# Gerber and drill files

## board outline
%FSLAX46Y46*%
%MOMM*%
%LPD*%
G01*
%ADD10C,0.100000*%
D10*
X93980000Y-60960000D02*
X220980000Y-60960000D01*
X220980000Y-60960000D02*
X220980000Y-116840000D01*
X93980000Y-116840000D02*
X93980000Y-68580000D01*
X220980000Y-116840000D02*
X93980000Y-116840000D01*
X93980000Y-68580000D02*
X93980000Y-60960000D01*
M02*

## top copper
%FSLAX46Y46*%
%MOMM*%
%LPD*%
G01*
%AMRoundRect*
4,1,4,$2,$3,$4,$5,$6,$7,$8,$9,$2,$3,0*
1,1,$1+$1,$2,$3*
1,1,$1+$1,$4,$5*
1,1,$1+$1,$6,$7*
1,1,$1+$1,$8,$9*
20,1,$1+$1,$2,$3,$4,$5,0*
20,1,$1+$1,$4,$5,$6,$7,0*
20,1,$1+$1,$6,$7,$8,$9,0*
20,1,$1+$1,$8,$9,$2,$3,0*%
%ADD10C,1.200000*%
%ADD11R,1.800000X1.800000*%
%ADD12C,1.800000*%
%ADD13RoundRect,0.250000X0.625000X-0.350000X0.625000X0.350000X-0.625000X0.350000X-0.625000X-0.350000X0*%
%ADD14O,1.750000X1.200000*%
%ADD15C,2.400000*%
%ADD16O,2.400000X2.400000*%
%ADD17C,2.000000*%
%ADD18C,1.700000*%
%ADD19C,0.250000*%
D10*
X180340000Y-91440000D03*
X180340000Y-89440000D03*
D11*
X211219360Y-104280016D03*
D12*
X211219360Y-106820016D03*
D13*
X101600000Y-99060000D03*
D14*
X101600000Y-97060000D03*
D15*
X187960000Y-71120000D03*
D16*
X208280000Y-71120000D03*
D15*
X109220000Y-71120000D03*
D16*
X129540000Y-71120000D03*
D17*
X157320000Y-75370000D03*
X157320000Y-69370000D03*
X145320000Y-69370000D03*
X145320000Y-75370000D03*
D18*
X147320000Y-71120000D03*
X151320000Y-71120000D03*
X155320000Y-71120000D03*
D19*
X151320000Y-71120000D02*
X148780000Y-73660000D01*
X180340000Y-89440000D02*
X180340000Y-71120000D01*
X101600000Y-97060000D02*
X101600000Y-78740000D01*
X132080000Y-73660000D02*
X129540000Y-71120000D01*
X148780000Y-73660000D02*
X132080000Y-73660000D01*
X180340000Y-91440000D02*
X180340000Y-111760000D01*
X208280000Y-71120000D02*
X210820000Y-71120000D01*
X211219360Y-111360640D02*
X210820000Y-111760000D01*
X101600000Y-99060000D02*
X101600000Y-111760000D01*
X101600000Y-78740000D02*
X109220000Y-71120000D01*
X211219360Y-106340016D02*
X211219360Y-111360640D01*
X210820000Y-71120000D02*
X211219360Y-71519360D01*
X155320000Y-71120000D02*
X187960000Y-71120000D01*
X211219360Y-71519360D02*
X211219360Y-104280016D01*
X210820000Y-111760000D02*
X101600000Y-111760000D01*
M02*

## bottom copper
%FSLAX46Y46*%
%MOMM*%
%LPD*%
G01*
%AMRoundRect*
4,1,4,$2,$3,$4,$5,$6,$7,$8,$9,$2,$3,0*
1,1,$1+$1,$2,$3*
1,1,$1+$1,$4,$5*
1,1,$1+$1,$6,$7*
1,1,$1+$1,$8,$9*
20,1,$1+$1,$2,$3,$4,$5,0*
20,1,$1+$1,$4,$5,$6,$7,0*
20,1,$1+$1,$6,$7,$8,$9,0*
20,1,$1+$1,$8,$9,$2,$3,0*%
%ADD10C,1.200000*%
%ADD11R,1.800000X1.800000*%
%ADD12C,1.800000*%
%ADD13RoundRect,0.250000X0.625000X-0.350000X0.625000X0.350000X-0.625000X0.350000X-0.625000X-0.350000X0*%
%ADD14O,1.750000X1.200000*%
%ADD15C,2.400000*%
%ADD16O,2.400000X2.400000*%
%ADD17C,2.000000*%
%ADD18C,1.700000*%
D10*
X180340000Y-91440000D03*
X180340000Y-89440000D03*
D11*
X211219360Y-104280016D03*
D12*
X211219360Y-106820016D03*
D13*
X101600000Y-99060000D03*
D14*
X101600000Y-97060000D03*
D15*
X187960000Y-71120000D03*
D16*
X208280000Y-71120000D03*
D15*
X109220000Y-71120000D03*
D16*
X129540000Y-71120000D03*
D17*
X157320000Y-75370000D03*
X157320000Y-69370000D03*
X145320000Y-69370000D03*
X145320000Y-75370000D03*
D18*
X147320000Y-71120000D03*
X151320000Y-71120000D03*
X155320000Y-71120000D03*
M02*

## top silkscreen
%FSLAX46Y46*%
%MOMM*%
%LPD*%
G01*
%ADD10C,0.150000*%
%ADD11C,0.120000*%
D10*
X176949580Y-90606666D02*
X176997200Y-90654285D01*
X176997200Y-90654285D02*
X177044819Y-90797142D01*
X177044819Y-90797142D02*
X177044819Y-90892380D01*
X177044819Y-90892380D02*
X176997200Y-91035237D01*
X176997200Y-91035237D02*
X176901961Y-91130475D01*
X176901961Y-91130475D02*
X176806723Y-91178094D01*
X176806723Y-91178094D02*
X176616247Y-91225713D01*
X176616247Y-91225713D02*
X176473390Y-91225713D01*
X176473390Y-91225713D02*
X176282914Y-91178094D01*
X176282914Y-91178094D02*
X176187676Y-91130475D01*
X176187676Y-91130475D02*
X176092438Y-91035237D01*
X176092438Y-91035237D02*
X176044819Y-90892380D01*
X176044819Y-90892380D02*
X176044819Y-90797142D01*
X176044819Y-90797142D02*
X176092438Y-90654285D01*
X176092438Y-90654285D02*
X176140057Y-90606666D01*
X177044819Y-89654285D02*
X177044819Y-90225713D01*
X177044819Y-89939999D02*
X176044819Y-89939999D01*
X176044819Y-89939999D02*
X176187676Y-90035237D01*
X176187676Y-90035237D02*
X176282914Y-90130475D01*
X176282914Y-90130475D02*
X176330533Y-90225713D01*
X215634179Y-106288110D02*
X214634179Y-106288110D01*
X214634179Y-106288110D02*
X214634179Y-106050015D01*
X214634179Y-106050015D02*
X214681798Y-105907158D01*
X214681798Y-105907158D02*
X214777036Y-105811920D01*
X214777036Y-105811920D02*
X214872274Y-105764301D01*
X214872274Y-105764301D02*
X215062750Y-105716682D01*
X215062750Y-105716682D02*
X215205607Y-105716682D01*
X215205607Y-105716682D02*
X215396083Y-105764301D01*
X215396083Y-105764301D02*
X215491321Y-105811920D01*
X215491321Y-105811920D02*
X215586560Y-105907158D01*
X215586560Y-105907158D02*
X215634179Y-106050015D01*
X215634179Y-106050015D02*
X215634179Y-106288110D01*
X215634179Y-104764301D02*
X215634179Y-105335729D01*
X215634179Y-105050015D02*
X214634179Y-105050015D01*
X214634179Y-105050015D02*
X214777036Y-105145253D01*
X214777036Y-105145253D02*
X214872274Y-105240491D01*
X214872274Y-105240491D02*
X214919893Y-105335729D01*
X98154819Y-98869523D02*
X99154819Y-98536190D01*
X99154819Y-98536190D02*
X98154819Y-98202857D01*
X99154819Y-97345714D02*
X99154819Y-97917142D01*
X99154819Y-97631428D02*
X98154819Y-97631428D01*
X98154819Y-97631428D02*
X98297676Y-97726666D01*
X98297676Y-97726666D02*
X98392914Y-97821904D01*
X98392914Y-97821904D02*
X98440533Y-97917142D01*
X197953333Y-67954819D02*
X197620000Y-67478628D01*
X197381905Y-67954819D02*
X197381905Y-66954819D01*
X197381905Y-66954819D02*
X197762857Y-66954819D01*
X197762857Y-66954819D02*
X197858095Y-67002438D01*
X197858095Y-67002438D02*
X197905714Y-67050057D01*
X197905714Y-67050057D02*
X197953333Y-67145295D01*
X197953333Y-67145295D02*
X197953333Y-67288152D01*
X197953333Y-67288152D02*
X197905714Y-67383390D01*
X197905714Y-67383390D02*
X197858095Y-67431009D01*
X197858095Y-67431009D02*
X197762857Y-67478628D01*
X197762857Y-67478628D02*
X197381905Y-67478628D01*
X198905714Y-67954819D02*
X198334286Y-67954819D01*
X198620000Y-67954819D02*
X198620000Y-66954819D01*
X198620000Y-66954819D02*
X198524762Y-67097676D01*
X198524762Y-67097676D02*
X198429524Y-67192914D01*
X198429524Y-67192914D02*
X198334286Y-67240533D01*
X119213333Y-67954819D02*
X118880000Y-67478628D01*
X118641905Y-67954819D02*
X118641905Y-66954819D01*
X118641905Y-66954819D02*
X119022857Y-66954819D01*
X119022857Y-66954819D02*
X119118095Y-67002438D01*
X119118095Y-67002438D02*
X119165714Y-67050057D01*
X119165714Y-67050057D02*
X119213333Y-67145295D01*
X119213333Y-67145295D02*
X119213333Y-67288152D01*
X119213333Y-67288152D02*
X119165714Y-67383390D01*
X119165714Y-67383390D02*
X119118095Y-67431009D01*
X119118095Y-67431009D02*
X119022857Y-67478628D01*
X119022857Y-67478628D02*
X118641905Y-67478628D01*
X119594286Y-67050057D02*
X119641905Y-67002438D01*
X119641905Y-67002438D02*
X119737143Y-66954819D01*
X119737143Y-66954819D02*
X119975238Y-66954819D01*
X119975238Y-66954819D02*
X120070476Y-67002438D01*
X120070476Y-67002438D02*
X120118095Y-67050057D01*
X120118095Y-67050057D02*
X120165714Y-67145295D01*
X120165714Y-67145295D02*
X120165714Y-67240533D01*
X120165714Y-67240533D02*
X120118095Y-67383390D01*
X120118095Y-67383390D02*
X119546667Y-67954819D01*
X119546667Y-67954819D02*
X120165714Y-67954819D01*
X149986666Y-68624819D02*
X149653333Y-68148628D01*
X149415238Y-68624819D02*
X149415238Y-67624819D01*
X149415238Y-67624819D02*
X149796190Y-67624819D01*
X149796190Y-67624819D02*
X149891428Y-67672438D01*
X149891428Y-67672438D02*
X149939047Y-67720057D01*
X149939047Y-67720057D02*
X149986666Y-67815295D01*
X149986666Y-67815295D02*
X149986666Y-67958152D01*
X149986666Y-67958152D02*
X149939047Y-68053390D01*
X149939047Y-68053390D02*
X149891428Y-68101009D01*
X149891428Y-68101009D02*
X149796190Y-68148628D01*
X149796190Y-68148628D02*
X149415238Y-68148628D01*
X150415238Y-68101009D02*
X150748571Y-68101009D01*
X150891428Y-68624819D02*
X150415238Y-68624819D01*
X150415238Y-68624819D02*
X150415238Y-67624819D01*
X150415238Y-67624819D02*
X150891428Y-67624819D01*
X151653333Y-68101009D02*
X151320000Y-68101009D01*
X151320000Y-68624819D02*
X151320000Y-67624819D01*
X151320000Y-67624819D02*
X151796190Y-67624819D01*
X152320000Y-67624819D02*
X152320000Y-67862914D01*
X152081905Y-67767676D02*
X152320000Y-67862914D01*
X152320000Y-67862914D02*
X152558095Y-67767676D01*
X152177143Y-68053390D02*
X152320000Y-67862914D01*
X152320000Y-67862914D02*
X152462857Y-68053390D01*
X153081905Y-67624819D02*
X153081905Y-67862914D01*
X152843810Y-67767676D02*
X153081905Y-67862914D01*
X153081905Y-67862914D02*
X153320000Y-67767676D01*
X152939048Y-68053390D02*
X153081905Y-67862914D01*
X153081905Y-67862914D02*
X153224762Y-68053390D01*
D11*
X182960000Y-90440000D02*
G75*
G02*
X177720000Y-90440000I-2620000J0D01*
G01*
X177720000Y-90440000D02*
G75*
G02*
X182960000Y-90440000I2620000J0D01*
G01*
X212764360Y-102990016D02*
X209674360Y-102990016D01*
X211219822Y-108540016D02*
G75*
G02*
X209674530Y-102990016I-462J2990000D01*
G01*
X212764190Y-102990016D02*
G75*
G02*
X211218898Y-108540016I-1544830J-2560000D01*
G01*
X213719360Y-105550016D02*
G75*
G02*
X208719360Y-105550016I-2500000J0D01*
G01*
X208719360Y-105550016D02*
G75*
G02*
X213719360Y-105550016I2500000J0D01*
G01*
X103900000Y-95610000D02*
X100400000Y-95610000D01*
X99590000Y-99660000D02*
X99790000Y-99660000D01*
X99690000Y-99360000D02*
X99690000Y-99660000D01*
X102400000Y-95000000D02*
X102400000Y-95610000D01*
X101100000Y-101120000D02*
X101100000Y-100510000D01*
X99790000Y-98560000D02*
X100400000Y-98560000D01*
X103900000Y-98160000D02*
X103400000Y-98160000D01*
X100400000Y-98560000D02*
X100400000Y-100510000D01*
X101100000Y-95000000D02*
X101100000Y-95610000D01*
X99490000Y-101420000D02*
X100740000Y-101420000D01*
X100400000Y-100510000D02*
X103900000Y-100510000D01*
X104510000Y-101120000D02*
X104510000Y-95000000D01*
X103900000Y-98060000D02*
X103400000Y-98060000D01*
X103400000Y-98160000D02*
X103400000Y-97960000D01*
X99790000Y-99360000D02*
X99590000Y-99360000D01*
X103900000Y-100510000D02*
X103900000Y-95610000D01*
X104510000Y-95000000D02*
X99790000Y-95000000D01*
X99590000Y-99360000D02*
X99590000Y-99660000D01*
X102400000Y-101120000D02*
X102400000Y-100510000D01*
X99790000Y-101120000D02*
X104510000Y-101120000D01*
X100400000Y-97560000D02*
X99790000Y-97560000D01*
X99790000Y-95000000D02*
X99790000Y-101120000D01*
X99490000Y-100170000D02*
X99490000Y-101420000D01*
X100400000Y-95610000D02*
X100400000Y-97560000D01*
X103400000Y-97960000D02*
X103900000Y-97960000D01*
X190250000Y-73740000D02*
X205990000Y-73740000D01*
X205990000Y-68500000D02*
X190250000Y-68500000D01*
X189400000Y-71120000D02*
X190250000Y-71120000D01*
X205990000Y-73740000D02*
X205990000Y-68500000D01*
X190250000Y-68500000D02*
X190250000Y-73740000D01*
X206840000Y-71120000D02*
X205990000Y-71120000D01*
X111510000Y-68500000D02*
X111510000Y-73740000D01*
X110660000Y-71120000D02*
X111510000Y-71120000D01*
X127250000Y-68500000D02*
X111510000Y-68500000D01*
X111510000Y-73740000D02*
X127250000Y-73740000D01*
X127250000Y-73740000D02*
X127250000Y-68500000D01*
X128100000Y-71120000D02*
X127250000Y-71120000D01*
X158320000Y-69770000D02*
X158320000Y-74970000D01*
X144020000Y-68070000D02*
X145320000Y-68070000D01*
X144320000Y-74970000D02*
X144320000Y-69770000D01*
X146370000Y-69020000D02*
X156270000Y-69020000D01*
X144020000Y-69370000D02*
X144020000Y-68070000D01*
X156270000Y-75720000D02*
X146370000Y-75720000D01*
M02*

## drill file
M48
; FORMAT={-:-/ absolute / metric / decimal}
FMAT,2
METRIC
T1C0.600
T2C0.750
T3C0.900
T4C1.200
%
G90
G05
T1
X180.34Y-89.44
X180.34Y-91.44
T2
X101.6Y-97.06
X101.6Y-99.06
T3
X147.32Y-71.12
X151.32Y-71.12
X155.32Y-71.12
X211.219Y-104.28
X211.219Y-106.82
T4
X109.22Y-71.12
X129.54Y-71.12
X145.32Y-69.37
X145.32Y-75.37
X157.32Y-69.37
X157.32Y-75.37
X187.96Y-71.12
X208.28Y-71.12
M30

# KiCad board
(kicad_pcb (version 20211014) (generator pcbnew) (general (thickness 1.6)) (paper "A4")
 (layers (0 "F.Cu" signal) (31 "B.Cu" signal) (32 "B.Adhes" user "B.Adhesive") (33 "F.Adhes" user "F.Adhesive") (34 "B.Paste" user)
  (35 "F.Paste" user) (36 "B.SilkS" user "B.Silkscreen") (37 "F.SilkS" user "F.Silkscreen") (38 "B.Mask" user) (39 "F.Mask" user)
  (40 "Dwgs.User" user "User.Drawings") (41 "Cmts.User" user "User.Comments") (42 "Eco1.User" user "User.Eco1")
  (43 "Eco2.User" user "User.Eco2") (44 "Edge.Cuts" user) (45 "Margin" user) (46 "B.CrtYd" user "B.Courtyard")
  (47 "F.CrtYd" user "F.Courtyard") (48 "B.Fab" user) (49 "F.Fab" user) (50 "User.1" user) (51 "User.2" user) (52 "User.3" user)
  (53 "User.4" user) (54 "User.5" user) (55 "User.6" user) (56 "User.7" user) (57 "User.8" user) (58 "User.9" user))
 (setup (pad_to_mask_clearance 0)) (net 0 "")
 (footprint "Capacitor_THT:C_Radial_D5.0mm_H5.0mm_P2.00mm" (layer "F.Cu") (at 180.34 91.44 90)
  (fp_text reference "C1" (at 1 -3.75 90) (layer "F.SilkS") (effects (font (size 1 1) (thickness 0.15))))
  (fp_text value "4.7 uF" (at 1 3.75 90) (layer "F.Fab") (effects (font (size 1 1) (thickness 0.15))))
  (fp_circle (center 1 0) (end 3.62 0) (layer "F.SilkS") (width 0.12) (fill none))
  (pad "1" thru_hole circle (at 0 0 90) (size 1.2 1.2) (drill 0.6) (layers *.Cu *.Mask))
  (pad "2" thru_hole circle (at 2 0 90) (size 1.2 1.2) (drill 0.6) (layers *.Cu *.Mask)))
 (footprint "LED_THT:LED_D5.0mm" (layer "F.Cu") (at 211.21936 104.280016 -90)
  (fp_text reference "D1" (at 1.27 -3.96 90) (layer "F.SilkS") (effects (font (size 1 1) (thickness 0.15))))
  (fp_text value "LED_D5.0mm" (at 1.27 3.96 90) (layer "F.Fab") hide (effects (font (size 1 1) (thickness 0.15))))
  (fp_line (start -1.29 -1.545) (end -1.29 1.545) (layer "F.SilkS") (width 0.12))
  (fp_arc (start 4.26 -0.000462) (mid 2.072002 2.880433) (end -1.29 1.54483) (layer "F.SilkS") (width 0.12))
  (fp_arc (start -1.29 -1.54483) (mid 2.072002 -2.880433) (end 4.26 0.000462) (layer "F.SilkS") (width 0.12))
  (fp_circle (center 1.27 0) (end 3.77 0) (layer "F.SilkS") (width 0.12) (fill none))
  (pad "1" thru_hole rect (at 0 0 270) (size 1.8 1.8) (drill 0.9) (layers *.Cu *.Mask))
  (pad "2" thru_hole circle (at 2.54 0 270) (size 1.8 1.8) (drill 0.9) (layers *.Cu *.Mask)))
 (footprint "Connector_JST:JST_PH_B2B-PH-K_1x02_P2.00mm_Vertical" (layer "F.Cu") (at 101.6 99.06 90)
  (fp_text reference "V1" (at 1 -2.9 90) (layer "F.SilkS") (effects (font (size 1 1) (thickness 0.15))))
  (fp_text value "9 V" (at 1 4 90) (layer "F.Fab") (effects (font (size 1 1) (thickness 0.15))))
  (fp_line (start 3.45 2.3) (end 3.45 -1.2) (layer "F.SilkS") (width 0.12))
  (fp_line (start -0.6 -2.01) (end -0.6 -1.81) (layer "F.SilkS") (width 0.12))
  (fp_line (start -0.3 -1.91) (end -0.6 -1.91) (layer "F.SilkS") (width 0.12))
  (fp_line (start 4.06 0.8) (end 3.45 0.8) (layer "F.SilkS") (width 0.12))
  (fp_line (start -2.06 -0.5) (end -1.45 -0.5) (layer "F.SilkS") (width 0.12))
  (fp_line (start 0.5 -1.81) (end 0.5 -1.2) (layer "F.SilkS") (width 0.12))
  (fp_line (start 0.9 2.3) (end 0.9 1.8) (layer "F.SilkS") (width 0.12))
  (fp_line (start 0.5 -1.2) (end -1.45 -1.2) (layer "F.SilkS") (width 0.12))
  (fp_line (start 4.06 -0.5) (end 3.45 -0.5) (layer "F.SilkS") (width 0.12))
  (fp_line (start -2.36 -2.11) (end -2.36 -0.86) (layer "F.SilkS") (width 0.12))
  (fp_line (start -1.45 -1.2) (end -1.45 2.3) (layer "F.SilkS") (width 0.12))
  (fp_line (start -2.06 2.91) (end 4.06 2.91) (layer "F.SilkS") (width 0.12))
  (fp_line (start 1 2.3) (end 1 1.8) (layer "F.SilkS") (width 0.12))
  (fp_line (start 0.9 1.8) (end 1.1 1.8) (layer "F.SilkS") (width 0.12))
  (fp_line (start -0.3 -1.81) (end -0.3 -2.01) (layer "F.SilkS") (width 0.12))
  (fp_line (start -1.45 2.3) (end 3.45 2.3) (layer "F.SilkS") (width 0.12))
  (fp_line (start 4.06 2.91) (end 4.06 -1.81) (layer "F.SilkS") (width 0.12))
  (fp_line (start -0.3 -2.01) (end -0.6 -2.01) (layer "F.SilkS") (width 0.12))
  (fp_line (start -2.06 0.8) (end -1.45 0.8) (layer "F.SilkS") (width 0.12))
  (fp_line (start -2.06 -1.81) (end -2.06 2.91) (layer "F.SilkS") (width 0.12))
  (fp_line (start 1.5 -1.2) (end 1.5 -1.81) (layer "F.SilkS") (width 0.12))
  (fp_line (start 4.06 -1.81) (end -2.06 -1.81) (layer "F.SilkS") (width 0.12))
  (fp_line (start -1.11 -2.11) (end -2.36 -2.11) (layer "F.SilkS") (width 0.12))
  (fp_line (start 3.45 -1.2) (end 1.5 -1.2) (layer "F.SilkS") (width 0.12))
  (fp_line (start 1.1 1.8) (end 1.1 2.3) (layer "F.SilkS") (width 0.12))
  (pad "1" thru_hole roundrect (at 0 0 90) (size 1.2 1.75) (drill 0.75) (layers *.Cu *.Mask) (roundrect_rratio 0.2083333333))
  (pad "2" thru_hole oval (at 2 0 90) (size 1.2 1.75) (drill 0.75) (layers *.Cu *.Mask)))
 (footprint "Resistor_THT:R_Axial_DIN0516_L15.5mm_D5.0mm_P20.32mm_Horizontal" (layer "F.Cu") (at 187.96 71.12)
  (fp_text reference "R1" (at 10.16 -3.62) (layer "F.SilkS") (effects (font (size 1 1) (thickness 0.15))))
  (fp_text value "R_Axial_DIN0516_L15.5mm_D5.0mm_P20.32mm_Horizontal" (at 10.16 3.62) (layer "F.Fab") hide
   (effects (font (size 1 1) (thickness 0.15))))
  (fp_line (start 2.29 2.62) (end 18.03 2.62) (layer "F.SilkS") (width 0.12))
  (fp_line (start 18.03 -2.62) (end 2.29 -2.62) (layer "F.SilkS") (width 0.12))
  (fp_line (start 1.44 0) (end 2.29 0) (layer "F.SilkS") (width 0.12))
  (fp_line (start 18.03 2.62) (end 18.03 -2.62) (layer "F.SilkS") (width 0.12))
  (fp_line (start 2.29 -2.62) (end 2.29 2.62) (layer "F.SilkS") (width 0.12))
  (fp_line (start 18.88 0) (end 18.03 0) (layer "F.SilkS") (width 0.12))
  (pad "1" thru_hole circle (at 0 0) (size 2.4 2.4) (drill 1.2) (layers *.Cu *.Mask))
  (pad "2" thru_hole oval (at 20.32 0) (size 2.4 2.4) (drill 1.2) (layers *.Cu *.Mask)))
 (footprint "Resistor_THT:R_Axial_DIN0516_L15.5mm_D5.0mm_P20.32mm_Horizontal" (layer "F.Cu") (at 109.22 71.12)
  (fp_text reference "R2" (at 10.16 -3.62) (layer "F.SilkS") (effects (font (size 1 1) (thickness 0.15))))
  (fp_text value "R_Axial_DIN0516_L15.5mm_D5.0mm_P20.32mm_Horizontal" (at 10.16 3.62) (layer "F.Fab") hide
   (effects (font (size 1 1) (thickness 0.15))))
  (fp_line (start 2.29 -2.62) (end 2.29 2.62) (layer "F.SilkS") (width 0.12))
  (fp_line (start 1.44 0) (end 2.29 0) (layer "F.SilkS") (width 0.12))
  (fp_line (start 18.03 -2.62) (end 2.29 -2.62) (layer "F.SilkS") (width 0.12))
  (fp_line (start 2.29 2.62) (end 18.03 2.62) (layer "F.SilkS") (width 0.12))
  (fp_line (start 18.03 2.62) (end 18.03 -2.62) (layer "F.SilkS") (width 0.12))
  (fp_line (start 18.88 0) (end 18.03 0) (layer "F.SilkS") (width 0.12))
  (pad "1" thru_hole circle (at 0 0) (size 2.4 2.4) (drill 1.2) (layers *.Cu *.Mask))
  (pad "2" thru_hole oval (at 20.32 0) (size 2.4 2.4) (drill 1.2) (layers *.Cu *.Mask)))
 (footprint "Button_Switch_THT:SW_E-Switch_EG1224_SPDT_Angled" (layer "F.Cu") (at 147.32 71.12)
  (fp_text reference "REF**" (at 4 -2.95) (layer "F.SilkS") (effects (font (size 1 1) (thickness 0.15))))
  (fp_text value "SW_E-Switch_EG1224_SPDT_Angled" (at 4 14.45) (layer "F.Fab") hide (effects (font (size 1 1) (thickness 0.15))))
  (fp_line (start 11 -1.35) (end 11 3.85) (layer "F.SilkS") (width 0.12))
  (fp_line (start -3.3 -3.05) (end -2 -3.05) (layer "F.SilkS") (width 0.12))
  (fp_line (start -3 3.85) (end -3 -1.35) (layer "F.SilkS") (width 0.12))
  (fp_line (start -0.95 -2.1) (end 8.95 -2.1) (layer "F.SilkS") (width 0.12))
  (fp_line (start -3.3 -1.75) (end -3.3 -3.05) (layer "F.SilkS") (width 0.12))
  (fp_line (start 8.95 4.6) (end -0.95 4.6) (layer "F.SilkS") (width 0.12))
  (pad "" thru_hole circle (at 10 4.25) (size 2 2) (drill 1.2) (layers *.Cu *.Mask))
  (pad "" thru_hole circle (at 10 -1.75) (size 2 2) (drill 1.2) (layers *.Cu *.Mask))
  (pad "" thru_hole circle (at -2 -1.75) (size 2 2) (drill 1.2) (layers *.Cu *.Mask))
  (pad "" thru_hole circle (at -2 4.25) (size 2 2) (drill 1.2) (layers *.Cu *.Mask))
  (pad "1" thru_hole circle (at 0 0) (size 1.7 1.7) (drill 0.9) (layers *.Cu *.Mask))
  (pad "2" thru_hole circle (at 4 0) (size 1.7 1.7) (drill 0.9) (layers *.Cu *.Mask))
  (pad "3" thru_hole circle (at 8 0) (size 1.7 1.7) (drill 0.9) (layers *.Cu *.Mask)))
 (gr_line (start 93.98 60.96) (end 220.98 60.96) (layer "Edge.Cuts") (width 0.1))
 (gr_line (start 220.98 60.96) (end 220.98 116.84) (layer "Edge.Cuts") (width 0.1))
 (gr_line (start 93.98 116.84) (end 93.98 68.58) (layer "Edge.Cuts") (width 0.1))
 (gr_line (start 220.98 116.84) (end 93.98 116.84) (layer "Edge.Cuts") (width 0.1))
 (gr_line (start 93.98 68.58) (end 93.98 60.96) (layer "Edge.Cuts") (width 0.1))
 (segment (start 151.32 71.12) (end 148.78 73.66) (width 0.25) (layer "F.Cu") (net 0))
 (segment (start 180.34 89.44) (end 180.34 71.12) (width 0.25) (layer "F.Cu") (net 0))
 (segment (start 101.6 97.06) (end 101.6 78.74) (width 0.25) (layer "F.Cu") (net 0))
 (segment (start 132.08 73.66) (end 129.54 71.12) (width 0.25) (layer "F.Cu") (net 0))
 (segment (start 148.78 73.66) (end 132.08 73.66) (width 0.25) (layer "F.Cu") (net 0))
 (segment (start 180.34 91.44) (end 180.34 111.76) (width 0.25) (layer "F.Cu") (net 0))
 (segment (start 208.28 71.12) (end 210.82 71.12) (width 0.25) (layer "F.Cu") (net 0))
 (segment (start 211.21936 111.36064) (end 210.82 111.76) (width 0.25) (layer "F.Cu") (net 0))
 (segment (start 101.6 99.06) (end 101.6 111.76) (width 0.25) (layer "F.Cu") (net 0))
 (segment (start 101.6 78.74) (end 109.22 71.12) (width 0.25) (layer "F.Cu") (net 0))
 (segment (start 211.21936 106.340016) (end 211.21936 111.36064) (width 0.25) (layer "F.Cu") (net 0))
 (segment (start 210.82 71.12) (end 211.21936 71.51936) (width 0.25) (layer "F.Cu") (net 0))
 (segment (start 155.32 71.12) (end 187.96 71.12) (width 0.25) (layer "F.Cu") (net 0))
 (segment (start 211.21936 71.51936) (end 211.21936 104.280016) (width 0.25) (layer "F.Cu") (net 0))
 (segment (start 210.82 111.76) (end 101.6 111.76) (width 0.25) (layer "F.Cu") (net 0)))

